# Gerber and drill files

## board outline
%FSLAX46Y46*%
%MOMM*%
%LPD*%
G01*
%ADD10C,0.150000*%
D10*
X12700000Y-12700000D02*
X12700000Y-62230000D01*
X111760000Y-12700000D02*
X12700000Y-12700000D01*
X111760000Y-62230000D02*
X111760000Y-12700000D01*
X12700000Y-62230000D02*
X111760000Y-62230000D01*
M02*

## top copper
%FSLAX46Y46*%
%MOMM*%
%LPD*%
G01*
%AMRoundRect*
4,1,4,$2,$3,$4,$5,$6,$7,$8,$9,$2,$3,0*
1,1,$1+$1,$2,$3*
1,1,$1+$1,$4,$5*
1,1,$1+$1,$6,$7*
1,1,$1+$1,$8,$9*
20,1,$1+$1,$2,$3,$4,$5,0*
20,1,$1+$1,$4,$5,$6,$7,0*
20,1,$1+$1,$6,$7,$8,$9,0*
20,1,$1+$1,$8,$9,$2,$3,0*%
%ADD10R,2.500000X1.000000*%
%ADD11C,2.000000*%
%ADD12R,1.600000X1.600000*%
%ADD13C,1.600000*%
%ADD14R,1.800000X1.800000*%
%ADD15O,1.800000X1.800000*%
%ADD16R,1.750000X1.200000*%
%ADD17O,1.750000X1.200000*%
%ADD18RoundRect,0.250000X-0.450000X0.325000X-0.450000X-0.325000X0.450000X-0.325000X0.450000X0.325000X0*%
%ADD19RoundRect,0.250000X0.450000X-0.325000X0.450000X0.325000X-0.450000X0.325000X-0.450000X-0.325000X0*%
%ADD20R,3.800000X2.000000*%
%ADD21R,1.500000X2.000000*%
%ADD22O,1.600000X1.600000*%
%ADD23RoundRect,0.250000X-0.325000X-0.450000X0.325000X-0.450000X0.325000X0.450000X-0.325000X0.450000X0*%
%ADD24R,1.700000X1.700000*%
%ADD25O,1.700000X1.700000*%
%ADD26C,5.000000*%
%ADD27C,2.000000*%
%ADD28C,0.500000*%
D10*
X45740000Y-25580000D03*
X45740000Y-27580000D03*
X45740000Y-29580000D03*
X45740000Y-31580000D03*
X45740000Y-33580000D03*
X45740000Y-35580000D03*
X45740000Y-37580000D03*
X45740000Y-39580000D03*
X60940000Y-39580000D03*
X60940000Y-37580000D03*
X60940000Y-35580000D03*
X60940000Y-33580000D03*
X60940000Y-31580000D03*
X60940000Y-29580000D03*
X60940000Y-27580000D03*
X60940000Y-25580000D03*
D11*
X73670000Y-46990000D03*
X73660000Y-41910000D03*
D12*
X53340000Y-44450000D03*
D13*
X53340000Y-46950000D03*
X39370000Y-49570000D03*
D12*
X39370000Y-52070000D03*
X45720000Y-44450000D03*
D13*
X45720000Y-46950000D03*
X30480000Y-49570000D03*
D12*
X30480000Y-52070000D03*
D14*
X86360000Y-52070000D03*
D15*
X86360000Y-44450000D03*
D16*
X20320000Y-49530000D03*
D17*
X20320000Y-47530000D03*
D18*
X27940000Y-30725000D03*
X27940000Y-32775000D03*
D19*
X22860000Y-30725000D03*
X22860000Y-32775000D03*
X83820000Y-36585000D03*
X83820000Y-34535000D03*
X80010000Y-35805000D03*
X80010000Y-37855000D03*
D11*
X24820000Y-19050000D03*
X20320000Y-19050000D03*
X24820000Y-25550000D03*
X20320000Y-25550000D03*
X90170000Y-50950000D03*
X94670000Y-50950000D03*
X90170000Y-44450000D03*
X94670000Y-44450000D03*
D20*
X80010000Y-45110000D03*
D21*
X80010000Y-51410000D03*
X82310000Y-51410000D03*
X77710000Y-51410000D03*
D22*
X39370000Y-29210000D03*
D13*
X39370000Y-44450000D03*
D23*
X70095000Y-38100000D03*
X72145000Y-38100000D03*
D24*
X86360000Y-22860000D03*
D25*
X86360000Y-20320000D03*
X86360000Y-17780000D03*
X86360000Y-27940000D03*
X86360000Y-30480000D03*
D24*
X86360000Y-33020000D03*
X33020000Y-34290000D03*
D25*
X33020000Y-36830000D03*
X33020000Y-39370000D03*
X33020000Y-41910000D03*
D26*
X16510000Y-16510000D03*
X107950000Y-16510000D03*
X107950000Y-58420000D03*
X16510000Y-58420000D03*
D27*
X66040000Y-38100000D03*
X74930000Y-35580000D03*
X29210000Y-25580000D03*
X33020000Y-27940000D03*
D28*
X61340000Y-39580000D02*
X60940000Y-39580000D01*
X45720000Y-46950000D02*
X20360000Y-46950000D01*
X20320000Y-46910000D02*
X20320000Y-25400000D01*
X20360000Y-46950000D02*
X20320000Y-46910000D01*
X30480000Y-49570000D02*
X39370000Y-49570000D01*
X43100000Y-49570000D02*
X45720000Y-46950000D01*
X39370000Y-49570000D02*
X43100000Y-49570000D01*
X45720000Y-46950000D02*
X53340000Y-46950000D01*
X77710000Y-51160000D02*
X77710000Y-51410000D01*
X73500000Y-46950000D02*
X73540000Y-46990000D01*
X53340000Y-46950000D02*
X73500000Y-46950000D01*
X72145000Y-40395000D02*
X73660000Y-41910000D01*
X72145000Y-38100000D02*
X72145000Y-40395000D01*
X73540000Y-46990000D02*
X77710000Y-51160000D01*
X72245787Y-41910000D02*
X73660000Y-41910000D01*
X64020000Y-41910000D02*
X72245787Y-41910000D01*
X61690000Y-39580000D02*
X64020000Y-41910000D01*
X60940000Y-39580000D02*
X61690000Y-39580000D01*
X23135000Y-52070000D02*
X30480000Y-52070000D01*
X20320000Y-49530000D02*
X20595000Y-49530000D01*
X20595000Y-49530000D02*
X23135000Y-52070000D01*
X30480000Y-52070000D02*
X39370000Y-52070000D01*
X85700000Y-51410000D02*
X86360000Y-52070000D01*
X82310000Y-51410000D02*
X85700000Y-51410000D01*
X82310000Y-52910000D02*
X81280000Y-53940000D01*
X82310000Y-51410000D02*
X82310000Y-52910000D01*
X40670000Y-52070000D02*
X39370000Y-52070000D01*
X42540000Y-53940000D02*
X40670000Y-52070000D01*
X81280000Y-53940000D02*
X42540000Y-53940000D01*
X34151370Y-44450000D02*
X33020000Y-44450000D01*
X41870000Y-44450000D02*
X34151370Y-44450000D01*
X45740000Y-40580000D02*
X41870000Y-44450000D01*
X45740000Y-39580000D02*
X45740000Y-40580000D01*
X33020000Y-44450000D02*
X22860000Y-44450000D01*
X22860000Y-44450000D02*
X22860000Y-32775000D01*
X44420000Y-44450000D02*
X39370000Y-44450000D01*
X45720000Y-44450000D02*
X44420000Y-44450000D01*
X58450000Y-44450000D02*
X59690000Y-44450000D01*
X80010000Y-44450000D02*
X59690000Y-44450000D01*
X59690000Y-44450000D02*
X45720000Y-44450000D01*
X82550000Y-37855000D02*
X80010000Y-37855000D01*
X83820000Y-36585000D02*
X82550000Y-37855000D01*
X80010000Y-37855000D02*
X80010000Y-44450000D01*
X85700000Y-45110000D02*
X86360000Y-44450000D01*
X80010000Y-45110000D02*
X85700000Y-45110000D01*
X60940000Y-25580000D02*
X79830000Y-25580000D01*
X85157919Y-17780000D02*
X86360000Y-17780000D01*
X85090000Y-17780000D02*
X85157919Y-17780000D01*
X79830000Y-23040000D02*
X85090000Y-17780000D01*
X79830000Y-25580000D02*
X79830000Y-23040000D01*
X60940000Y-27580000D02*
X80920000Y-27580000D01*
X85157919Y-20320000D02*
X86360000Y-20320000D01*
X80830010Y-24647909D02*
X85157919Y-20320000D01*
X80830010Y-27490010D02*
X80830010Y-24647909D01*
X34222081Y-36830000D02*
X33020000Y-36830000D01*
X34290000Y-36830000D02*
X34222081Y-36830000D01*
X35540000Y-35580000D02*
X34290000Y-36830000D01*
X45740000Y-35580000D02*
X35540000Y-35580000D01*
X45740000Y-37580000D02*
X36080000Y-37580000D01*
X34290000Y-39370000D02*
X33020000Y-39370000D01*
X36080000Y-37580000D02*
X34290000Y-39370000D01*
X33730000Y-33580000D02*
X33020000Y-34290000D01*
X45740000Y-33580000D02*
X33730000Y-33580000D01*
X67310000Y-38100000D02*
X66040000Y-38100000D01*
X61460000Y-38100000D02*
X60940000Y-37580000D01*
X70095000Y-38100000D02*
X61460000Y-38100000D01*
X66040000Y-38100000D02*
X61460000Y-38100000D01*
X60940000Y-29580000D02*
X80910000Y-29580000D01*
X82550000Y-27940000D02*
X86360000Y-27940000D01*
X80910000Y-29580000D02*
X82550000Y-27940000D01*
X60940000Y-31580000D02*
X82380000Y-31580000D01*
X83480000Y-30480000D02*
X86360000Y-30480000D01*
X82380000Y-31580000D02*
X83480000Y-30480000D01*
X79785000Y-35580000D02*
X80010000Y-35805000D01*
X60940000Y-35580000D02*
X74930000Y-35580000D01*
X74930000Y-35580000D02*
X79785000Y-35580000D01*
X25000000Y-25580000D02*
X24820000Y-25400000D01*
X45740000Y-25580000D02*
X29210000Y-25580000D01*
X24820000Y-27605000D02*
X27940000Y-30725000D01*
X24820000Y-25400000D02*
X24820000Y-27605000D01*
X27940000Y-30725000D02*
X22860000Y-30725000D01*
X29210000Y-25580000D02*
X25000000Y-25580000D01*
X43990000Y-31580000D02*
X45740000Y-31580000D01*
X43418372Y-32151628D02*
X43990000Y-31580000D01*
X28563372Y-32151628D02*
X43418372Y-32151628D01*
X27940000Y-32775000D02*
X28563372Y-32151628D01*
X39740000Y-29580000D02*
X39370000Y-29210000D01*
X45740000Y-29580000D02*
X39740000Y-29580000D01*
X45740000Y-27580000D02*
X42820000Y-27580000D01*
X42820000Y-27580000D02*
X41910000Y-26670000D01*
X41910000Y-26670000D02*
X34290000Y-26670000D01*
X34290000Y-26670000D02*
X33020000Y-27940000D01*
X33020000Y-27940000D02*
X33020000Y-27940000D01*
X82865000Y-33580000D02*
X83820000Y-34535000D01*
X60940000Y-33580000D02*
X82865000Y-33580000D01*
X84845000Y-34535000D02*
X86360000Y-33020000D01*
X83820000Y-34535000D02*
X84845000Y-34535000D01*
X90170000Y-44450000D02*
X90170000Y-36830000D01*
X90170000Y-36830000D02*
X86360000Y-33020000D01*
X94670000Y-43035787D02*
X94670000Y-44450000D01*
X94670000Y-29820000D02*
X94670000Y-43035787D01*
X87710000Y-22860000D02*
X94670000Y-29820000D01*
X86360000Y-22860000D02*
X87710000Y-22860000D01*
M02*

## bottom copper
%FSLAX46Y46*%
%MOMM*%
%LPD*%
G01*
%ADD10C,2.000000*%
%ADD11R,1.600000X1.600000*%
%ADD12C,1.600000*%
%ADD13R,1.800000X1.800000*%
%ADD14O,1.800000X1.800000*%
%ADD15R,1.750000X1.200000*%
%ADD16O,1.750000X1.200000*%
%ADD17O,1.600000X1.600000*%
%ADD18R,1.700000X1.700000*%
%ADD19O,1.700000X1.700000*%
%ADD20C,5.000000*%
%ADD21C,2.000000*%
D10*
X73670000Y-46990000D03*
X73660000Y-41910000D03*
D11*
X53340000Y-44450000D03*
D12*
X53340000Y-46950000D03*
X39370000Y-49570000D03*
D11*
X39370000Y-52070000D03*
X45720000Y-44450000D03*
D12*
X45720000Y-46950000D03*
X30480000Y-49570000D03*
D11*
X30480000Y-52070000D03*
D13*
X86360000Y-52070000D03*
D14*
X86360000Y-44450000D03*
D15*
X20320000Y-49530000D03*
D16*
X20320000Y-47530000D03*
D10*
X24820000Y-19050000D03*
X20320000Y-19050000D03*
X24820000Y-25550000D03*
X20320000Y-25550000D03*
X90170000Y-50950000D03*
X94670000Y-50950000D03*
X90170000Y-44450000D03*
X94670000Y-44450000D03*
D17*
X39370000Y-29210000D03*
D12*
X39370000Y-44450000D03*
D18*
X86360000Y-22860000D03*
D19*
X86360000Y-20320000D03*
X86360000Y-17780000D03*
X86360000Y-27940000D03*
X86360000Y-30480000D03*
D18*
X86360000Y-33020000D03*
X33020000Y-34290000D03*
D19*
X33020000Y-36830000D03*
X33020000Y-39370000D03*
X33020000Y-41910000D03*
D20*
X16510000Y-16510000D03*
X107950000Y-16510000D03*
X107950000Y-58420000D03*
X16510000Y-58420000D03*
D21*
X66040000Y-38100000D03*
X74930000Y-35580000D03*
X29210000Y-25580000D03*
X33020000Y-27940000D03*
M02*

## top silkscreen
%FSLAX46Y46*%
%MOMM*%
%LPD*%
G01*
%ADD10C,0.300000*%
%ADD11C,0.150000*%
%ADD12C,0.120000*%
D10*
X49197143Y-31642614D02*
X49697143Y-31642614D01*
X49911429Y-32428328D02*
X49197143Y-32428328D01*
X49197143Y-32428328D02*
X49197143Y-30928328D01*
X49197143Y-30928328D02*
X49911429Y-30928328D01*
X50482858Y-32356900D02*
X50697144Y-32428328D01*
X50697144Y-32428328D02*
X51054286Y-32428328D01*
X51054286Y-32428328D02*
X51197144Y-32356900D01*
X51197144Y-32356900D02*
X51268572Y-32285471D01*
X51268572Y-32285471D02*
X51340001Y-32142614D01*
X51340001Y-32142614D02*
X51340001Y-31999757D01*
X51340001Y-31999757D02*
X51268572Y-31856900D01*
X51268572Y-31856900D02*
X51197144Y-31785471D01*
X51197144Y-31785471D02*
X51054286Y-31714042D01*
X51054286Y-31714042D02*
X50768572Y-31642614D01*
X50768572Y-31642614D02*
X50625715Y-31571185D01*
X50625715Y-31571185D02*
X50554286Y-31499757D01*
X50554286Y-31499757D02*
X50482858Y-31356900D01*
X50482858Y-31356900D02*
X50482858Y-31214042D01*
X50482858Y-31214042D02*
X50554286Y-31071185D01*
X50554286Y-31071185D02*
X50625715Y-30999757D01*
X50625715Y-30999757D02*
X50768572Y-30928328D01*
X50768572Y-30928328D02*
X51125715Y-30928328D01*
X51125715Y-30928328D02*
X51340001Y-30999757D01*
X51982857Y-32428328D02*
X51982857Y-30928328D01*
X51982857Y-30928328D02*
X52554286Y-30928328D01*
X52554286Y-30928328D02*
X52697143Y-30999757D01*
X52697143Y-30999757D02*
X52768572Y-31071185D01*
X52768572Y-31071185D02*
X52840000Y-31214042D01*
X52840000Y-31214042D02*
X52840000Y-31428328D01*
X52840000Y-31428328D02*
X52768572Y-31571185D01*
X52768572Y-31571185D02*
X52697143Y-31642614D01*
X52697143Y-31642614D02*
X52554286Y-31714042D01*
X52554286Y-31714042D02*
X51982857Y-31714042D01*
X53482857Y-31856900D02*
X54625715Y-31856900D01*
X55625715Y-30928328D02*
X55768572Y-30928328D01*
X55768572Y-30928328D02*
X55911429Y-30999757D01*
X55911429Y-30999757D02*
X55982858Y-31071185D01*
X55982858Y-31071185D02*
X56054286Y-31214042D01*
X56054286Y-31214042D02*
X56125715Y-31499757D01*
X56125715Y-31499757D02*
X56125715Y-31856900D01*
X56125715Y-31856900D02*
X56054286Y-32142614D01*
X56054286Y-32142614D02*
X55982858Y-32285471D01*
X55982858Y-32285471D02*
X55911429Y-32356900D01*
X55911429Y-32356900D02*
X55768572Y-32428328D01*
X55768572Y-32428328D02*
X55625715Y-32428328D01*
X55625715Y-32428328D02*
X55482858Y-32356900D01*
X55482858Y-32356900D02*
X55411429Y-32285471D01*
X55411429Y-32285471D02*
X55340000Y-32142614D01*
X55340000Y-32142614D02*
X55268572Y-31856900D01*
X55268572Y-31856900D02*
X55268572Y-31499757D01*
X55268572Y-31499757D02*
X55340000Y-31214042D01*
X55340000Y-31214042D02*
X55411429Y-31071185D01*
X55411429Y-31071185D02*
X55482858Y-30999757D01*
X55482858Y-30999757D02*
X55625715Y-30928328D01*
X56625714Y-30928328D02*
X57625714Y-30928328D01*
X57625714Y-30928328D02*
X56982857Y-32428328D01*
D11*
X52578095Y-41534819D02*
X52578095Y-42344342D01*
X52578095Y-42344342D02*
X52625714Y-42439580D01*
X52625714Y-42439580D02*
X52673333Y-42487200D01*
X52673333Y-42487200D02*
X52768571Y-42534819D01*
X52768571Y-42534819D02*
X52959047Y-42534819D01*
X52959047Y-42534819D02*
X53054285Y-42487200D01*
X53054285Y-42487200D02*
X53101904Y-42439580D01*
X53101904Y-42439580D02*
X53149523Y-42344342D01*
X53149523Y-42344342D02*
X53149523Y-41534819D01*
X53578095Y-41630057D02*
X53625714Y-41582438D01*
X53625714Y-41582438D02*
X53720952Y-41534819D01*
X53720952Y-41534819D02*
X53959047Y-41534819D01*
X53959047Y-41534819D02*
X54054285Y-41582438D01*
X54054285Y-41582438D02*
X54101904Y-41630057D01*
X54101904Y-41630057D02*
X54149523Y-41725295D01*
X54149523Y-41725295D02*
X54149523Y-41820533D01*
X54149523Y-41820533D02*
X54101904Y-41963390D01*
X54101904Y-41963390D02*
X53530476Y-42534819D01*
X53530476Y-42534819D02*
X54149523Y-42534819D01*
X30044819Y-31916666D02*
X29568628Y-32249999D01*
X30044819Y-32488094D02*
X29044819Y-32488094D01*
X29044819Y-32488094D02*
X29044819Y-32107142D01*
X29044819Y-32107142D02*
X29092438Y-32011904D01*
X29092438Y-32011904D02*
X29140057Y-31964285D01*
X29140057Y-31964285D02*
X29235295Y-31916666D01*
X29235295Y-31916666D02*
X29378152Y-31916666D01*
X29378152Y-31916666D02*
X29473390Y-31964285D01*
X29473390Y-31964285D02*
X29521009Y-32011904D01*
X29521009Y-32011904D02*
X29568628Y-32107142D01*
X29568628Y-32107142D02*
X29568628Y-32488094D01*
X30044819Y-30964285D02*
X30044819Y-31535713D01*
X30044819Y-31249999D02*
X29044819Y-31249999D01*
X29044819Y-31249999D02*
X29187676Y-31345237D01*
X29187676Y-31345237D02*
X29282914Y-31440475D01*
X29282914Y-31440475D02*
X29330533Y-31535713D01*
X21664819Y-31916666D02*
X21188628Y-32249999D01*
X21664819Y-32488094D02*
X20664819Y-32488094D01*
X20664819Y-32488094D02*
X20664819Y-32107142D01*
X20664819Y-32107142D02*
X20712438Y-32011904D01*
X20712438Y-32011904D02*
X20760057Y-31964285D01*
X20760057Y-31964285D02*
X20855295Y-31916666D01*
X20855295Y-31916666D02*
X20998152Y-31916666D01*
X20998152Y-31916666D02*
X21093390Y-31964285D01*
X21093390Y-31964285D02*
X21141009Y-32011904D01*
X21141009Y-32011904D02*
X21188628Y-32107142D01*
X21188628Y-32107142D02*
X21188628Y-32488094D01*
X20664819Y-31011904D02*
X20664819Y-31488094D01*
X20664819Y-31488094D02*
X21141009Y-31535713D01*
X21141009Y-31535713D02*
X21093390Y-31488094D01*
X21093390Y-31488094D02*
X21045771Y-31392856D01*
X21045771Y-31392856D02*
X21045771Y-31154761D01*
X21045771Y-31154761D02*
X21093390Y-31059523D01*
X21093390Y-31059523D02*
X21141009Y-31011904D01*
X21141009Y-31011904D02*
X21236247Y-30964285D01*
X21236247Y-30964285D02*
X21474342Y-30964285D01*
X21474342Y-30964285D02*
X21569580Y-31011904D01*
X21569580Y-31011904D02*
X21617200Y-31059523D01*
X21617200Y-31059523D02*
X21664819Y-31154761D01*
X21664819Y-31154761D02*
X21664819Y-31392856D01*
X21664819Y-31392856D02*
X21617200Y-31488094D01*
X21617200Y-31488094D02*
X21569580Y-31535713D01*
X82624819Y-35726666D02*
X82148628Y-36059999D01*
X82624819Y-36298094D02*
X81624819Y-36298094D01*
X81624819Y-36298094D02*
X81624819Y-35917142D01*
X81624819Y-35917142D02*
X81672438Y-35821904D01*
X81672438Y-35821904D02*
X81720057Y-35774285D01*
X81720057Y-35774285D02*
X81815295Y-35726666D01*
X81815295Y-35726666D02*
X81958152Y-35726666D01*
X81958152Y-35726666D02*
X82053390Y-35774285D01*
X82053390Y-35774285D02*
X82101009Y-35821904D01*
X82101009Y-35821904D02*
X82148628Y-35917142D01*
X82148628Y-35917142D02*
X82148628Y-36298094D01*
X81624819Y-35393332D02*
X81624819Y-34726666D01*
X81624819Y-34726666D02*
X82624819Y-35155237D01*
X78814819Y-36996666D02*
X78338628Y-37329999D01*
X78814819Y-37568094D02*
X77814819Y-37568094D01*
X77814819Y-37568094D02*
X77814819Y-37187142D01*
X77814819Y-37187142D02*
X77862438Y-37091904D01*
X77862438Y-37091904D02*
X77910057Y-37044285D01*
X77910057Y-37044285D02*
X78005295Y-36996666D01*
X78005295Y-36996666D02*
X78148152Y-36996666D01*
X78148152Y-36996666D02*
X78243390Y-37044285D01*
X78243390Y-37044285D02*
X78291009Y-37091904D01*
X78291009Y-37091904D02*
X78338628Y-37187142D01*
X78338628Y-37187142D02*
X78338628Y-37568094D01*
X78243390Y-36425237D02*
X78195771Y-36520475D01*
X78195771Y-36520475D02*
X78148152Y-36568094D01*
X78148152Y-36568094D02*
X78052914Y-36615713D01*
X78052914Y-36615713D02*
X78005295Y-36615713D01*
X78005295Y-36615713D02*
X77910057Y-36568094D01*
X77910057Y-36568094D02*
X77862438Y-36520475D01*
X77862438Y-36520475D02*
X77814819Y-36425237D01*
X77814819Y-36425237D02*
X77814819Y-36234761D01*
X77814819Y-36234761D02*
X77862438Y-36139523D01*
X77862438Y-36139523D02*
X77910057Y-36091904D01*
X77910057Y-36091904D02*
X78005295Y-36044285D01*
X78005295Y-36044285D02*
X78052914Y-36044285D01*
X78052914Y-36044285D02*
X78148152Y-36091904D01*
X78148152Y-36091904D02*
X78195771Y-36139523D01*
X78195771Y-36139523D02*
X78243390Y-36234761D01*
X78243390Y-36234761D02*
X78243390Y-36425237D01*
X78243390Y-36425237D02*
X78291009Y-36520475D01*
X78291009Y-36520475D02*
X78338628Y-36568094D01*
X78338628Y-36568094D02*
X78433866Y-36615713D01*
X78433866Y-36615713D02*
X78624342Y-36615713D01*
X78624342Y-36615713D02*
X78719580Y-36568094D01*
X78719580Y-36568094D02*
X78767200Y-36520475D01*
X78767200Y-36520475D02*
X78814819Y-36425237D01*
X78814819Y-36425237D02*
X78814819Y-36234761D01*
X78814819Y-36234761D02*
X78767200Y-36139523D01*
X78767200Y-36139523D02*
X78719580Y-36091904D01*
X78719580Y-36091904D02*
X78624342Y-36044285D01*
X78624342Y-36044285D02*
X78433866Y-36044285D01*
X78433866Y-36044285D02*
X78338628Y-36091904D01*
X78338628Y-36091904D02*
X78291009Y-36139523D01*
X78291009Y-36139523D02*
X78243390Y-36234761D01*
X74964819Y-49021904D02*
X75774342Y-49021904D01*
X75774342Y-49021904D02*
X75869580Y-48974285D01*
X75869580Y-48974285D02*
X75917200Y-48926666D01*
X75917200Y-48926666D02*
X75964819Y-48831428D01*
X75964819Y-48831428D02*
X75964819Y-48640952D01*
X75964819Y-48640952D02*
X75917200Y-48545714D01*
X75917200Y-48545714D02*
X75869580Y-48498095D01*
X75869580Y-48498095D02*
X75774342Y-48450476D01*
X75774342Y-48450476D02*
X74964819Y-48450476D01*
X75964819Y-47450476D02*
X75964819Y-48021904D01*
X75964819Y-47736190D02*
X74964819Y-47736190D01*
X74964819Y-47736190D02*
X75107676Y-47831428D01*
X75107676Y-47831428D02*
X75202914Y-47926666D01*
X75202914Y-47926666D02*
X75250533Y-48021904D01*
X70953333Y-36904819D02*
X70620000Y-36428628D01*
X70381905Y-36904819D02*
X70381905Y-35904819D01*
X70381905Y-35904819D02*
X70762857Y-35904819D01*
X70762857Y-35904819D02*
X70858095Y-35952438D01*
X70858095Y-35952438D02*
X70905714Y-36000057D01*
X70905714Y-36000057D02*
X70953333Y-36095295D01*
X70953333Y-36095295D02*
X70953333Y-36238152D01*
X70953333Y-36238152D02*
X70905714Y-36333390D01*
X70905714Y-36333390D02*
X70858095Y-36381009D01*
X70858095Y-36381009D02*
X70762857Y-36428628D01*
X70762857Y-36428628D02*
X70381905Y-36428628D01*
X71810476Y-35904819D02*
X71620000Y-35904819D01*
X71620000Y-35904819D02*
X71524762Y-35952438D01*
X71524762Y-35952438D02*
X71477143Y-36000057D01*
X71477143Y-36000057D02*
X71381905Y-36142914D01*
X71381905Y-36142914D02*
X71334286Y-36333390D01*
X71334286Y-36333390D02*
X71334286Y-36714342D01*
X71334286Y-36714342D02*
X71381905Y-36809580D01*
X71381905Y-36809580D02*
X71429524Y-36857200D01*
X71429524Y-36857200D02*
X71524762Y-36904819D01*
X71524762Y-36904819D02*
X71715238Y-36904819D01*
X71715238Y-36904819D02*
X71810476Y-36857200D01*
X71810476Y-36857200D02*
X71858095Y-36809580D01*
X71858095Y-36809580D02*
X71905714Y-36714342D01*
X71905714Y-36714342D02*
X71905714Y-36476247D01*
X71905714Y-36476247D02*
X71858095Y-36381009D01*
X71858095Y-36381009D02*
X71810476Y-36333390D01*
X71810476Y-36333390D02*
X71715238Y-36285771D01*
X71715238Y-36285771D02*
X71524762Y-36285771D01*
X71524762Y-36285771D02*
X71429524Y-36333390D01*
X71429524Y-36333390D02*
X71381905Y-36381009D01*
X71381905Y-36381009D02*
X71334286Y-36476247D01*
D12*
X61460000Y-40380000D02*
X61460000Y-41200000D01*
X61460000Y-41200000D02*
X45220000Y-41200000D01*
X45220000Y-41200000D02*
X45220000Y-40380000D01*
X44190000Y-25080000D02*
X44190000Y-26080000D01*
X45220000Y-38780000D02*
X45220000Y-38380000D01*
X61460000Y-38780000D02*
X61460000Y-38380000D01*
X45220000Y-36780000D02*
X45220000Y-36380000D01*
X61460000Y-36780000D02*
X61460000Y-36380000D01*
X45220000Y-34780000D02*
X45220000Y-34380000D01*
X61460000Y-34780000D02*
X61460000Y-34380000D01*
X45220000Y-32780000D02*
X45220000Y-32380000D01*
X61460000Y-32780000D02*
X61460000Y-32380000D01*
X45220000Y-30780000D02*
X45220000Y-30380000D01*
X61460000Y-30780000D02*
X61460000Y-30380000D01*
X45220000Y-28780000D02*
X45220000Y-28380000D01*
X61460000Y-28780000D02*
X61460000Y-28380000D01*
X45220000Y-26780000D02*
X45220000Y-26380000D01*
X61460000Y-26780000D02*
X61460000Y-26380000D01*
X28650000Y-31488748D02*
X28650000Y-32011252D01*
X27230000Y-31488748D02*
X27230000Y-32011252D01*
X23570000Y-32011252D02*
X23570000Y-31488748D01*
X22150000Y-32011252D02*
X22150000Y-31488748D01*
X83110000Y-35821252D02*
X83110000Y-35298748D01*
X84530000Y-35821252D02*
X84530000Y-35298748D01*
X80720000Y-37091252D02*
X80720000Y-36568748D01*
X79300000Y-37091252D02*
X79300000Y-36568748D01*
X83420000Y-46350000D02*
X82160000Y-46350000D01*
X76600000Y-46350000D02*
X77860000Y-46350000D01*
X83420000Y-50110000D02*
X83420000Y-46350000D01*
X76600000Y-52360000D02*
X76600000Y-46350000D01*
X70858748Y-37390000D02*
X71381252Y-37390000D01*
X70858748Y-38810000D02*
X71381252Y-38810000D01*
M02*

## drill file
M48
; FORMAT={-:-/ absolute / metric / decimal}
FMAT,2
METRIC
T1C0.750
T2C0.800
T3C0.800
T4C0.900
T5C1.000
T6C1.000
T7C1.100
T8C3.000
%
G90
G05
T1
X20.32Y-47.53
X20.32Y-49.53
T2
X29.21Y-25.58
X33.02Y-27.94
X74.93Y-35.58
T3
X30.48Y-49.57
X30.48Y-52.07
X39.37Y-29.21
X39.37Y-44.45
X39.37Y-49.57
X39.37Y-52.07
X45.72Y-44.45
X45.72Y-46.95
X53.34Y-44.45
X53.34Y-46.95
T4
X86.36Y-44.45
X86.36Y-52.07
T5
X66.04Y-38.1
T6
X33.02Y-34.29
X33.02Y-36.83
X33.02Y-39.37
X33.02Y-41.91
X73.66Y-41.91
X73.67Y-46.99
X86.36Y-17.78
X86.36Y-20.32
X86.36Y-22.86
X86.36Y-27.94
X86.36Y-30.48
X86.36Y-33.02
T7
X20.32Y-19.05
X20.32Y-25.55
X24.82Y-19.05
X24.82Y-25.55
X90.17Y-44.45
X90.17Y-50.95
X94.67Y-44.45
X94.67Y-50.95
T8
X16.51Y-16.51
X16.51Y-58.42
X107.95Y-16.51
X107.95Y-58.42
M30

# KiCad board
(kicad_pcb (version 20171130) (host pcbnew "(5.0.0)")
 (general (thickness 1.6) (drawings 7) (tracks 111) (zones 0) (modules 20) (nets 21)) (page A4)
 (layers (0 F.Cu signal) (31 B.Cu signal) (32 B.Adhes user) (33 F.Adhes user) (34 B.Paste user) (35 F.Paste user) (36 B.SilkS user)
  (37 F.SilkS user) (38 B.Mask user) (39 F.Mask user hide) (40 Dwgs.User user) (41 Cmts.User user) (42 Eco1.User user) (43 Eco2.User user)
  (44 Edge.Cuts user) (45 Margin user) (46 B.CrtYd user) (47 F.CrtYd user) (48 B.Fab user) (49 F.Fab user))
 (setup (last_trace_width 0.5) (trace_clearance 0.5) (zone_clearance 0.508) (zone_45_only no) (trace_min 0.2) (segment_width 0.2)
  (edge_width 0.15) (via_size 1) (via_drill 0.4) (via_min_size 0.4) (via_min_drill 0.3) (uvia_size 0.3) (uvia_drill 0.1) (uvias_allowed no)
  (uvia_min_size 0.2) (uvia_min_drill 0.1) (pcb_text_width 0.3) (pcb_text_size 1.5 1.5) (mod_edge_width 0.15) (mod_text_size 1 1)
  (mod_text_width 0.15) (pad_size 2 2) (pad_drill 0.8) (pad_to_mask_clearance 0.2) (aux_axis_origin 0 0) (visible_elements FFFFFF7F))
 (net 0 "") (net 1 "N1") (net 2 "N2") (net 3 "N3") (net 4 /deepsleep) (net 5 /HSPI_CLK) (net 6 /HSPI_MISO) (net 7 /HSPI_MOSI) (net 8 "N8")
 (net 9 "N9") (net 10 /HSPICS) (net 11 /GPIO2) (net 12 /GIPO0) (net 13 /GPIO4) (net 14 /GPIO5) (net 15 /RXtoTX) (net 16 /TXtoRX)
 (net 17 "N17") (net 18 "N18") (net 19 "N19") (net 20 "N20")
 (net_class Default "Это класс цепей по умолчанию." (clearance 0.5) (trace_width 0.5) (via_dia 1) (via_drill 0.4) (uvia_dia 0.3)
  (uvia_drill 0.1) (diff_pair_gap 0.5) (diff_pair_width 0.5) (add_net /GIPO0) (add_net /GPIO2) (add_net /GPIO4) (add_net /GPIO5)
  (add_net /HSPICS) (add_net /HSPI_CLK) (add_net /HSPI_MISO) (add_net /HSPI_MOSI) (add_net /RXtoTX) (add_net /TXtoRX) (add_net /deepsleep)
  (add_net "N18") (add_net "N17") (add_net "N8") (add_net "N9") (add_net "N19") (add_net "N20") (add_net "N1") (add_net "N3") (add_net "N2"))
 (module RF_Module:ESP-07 (layer F.Cu) (at 53.34 30.48)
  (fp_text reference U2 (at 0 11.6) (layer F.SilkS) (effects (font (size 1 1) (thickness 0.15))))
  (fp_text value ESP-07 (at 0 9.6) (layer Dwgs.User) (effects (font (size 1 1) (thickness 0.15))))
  (fp_line (start 8.12 9.9) (end 8.12 10.72) (layer F.SilkS) (width 0.12))
  (fp_line (start 8.12 10.72) (end -8.12 10.72) (layer F.SilkS) (width 0.12))
  (fp_line (start -8.12 10.72) (end -8.12 9.9) (layer F.SilkS) (width 0.12))
  (fp_line (start -9.15 -5.4) (end -9.15 -4.4) (layer F.SilkS) (width 0.12))
  (fp_line (start -8.12 8.3) (end -8.12 7.9) (layer F.SilkS) (width 0.12))
  (fp_line (start 8.12 8.3) (end 8.12 7.9) (layer F.SilkS) (width 0.12))
  (fp_line (start -8.12 6.3) (end -8.12 5.9) (layer F.SilkS) (width 0.12))
  (fp_line (start 8.12 6.3) (end 8.12 5.9) (layer F.SilkS) (width 0.12))
  (fp_line (start -8.12 4.3) (end -8.12 3.9) (layer F.SilkS) (width 0.12))
  (fp_line (start 8.12 4.3) (end 8.12 3.9) (layer F.SilkS) (width 0.12))
  (fp_line (start -8.12 2.3) (end -8.12 1.9) (layer F.SilkS) (width 0.12))
  (fp_line (start 8.12 2.3) (end 8.12 1.9) (layer F.SilkS) (width 0.12))
  (fp_line (start -8.12 0.3) (end -8.12 -0.1) (layer F.SilkS) (width 0.12))
  (fp_line (start 8.12 0.3) (end 8.12 -0.1) (layer F.SilkS) (width 0.12))
  (fp_line (start -8.12 -1.7) (end -8.12 -2.1) (layer F.SilkS) (width 0.12))
  (fp_line (start 8.12 -1.7) (end 8.12 -2.1) (layer F.SilkS) (width 0.12))
  (fp_line (start -8.12 -3.7) (end -8.12 -4.1) (layer F.SilkS) (width 0.12))
  (fp_line (start 8.12 -3.7) (end 8.12 -4.1) (layer F.SilkS) (width 0.12))
  (pad 1 smd rect (at -7.6 -4.9) (size 2.5 1) (layers F.Cu F.Paste F.Mask) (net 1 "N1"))
  (pad 2 smd rect (at -7.6 -2.9) (size 2.5 1) (layers F.Cu F.Paste F.Mask) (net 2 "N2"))
  (pad 3 smd rect (at -7.6 -0.9) (size 2.5 1) (layers F.Cu F.Paste F.Mask) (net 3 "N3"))
  (pad 4 smd rect (at -7.6 1.1) (size 2.5 1) (layers F.Cu F.Paste F.Mask) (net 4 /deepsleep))
  (pad 5 smd rect (at -7.6 3.1) (size 2.5 1) (layers F.Cu F.Paste F.Mask) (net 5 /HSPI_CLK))
  (pad 6 smd rect (at -7.6 5.1) (size 2.5 1) (layers F.Cu F.Paste F.Mask) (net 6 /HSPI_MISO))
  (pad 7 smd rect (at -7.6 7.1) (size 2.5 1) (layers F.Cu F.Paste F.Mask) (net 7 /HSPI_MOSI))
  (pad 8 smd rect (at -7.6 9.1) (size 2.5 1) (layers F.Cu F.Paste F.Mask) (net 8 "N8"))
  (pad 9 smd rect (at 7.6 9.1) (size 2.5 1) (layers F.Cu F.Paste F.Mask) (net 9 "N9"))
  (pad 10 smd rect (at 7.6 7.1) (size 2.5 1) (layers F.Cu F.Paste F.Mask) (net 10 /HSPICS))
  (pad 11 smd rect (at 7.6 5.1) (size 2.5 1) (layers F.Cu F.Paste F.Mask) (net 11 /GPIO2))
  (pad 12 smd rect (at 7.6 3.1) (size 2.5 1) (layers F.Cu F.Paste F.Mask) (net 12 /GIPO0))
  (pad 13 smd rect (at 7.6 1.1) (size 2.5 1) (layers F.Cu F.Paste F.Mask) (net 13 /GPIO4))
  (pad 14 smd rect (at 7.6 -0.9) (size 2.5 1) (layers F.Cu F.Paste F.Mask) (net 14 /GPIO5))
  (pad 15 smd rect (at 7.6 -2.9) (size 2.5 1) (layers F.Cu F.Paste F.Mask) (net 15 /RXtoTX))
  (pad 16 smd rect (at 7.6 -4.9) (size 2.5 1) (layers F.Cu F.Paste F.Mask) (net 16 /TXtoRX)))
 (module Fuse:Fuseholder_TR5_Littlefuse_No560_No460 (layer B.Cu) (at 73.66 41.91 270)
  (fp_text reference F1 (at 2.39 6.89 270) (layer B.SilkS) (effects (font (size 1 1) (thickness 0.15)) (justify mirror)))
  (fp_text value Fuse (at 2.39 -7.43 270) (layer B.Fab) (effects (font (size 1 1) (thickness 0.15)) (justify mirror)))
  (pad 2 thru_hole circle (at 5.08 -0.01 270) (size 2 2) (drill 1) (layers *.Cu *.Mask) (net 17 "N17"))
  (pad 1 thru_hole circle (at 0 0 270) (size 2 2) (drill 1) (layers *.Cu *.Mask) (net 9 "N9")))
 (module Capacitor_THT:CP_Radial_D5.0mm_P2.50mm (layer B.Cu) (at 53.34 44.45 270)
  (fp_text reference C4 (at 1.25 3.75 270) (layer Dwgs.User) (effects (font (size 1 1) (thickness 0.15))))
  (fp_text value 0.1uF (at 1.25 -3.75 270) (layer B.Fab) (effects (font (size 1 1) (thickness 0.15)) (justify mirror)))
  (pad 1 thru_hole rect (at 0 0 270) (size 1.6 1.6) (drill 0.8) (layers *.Cu *.Mask) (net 8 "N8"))
  (pad 2 thru_hole circle (at 2.5 0 270) (size 1.6 1.6) (drill 0.8) (layers *.Cu *.Mask) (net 17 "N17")))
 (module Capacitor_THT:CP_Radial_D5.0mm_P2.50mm (layer B.Cu) (at 39.37 52.07 90)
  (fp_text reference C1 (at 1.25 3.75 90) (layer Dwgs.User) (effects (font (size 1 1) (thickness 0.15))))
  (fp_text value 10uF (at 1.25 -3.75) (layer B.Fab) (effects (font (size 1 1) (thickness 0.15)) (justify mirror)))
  (pad 2 thru_hole circle (at 2.5 0 90) (size 1.6 1.6) (drill 0.8) (layers *.Cu *.Mask) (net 17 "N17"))
  (pad 1 thru_hole rect (at 0 0 90) (size 1.6 1.6) (drill 0.8) (layers *.Cu *.Mask) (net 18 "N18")))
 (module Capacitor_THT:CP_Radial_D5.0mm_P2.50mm (layer B.Cu) (at 45.72 44.45 270)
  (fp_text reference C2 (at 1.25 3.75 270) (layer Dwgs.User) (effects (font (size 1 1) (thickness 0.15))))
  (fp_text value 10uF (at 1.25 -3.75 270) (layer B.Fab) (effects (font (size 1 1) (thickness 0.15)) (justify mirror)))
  (pad 1 thru_hole rect (at 0 0 270) (size 1.6 1.6) (drill 0.8) (layers *.Cu *.Mask) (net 8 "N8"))
  (pad 2 thru_hole circle (at 2.5 0 270) (size 1.6 1.6) (drill 0.8) (layers *.Cu *.Mask) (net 17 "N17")))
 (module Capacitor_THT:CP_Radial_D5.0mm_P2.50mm (layer B.Cu) (at 30.48 52.07 90)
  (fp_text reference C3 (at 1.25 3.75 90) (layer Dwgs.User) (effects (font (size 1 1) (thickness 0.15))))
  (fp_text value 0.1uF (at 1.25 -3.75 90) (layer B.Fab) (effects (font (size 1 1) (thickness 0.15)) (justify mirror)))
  (pad 2 thru_hole circle (at 2.5 0 90) (size 1.6 1.6) (drill 0.8) (layers *.Cu *.Mask) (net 17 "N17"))
  (pad 1 thru_hole rect (at 0 0 90) (size 1.6 1.6) (drill 0.8) (layers *.Cu *.Mask) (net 18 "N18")))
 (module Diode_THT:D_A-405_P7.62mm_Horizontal (layer B.Cu) (at 86.36 52.07 90)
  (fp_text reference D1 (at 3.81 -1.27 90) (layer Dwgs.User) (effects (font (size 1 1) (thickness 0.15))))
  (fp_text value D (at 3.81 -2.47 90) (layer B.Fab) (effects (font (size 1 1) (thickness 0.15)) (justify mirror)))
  (pad 1 thru_hole rect (at 0 0 90) (size 1.8 1.8) (drill 0.9) (layers *.Cu *.Mask) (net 18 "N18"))
  (pad 2 thru_hole oval (at 7.62 0 90) (size 1.8 1.8) (drill 0.9) (layers *.Cu *.Mask) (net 8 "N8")))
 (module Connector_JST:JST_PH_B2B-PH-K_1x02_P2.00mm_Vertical (layer B.Cu) (at 20.32 49.53 90)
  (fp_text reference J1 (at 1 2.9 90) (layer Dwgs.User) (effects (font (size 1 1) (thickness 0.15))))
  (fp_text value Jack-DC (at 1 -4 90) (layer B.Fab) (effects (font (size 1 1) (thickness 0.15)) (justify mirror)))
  (pad 1 thru_hole rect (at 0 0 90) (size 1.2 1.75) (drill 0.75) (layers *.Cu *.Mask) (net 18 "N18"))
  (pad 2 thru_hole oval (at 2 0 90) (size 1.2 1.75) (drill 0.75) (layers *.Cu *.Mask) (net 17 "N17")))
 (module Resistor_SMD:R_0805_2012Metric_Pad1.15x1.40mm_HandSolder (layer F.Cu) (at 27.94 31.75 270)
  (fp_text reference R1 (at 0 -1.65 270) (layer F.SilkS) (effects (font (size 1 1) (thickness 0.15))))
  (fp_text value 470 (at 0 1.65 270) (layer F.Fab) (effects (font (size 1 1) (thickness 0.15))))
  (fp_line (start -0.261252 -0.71) (end 0.261252 -0.71) (layer F.SilkS) (width 0.12))
  (fp_line (start -0.261252 0.71) (end 0.261252 0.71) (layer F.SilkS) (width 0.12))
  (pad 1 smd roundrect (at -1.025 0 270) (size 1.15 1.4) (layers F.Cu F.Paste F.Mask) (roundrect_rratio 0.217391) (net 1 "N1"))
  (pad 2 smd roundrect (at 1.025 0 270) (size 1.15 1.4) (layers F.Cu F.Paste F.Mask) (roundrect_rratio 0.217391) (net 4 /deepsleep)))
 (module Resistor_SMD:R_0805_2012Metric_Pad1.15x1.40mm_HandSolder (layer F.Cu) (at 22.86 31.75 90)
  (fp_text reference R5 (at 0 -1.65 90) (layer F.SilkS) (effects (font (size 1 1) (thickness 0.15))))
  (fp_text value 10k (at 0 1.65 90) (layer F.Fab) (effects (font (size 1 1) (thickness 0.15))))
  (fp_line (start -0.261252 0.71) (end 0.261252 0.71) (layer F.SilkS) (width 0.12))
  (fp_line (start -0.261252 -0.71) (end 0.261252 -0.71) (layer F.SilkS) (width 0.12))
  (pad 2 smd roundrect (at 1.025 0 90) (size 1.15 1.4) (layers F.Cu F.Paste F.Mask) (roundrect_rratio 0.217391) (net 1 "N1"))
  (pad 1 smd roundrect (at -1.025 0 90) (size 1.15 1.4) (layers F.Cu F.Paste F.Mask) (roundrect_rratio 0.217391) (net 8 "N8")))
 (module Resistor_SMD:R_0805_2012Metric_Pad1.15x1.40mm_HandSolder (layer F.Cu) (at 83.82 35.56 90)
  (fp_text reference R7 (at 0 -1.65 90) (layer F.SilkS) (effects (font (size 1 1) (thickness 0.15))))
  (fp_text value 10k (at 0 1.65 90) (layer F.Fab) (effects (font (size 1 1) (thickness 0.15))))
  (fp_line (start -0.261252 -0.71) (end 0.261252 -0.71) (layer F.SilkS) (width 0.12))
  (fp_line (start -0.261252 0.71) (end 0.261252 0.71) (layer F.SilkS) (width 0.12))
  (pad 1 smd roundrect (at -1.025 0 90) (size 1.15 1.4) (layers F.Cu F.Paste F.Mask) (roundrect_rratio 0.217391) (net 8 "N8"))
  (pad 2 smd roundrect (at 1.025 0 90) (size 1.15 1.4) (layers F.Cu F.Paste F.Mask) (roundrect_rratio 0.217391) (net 12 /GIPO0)))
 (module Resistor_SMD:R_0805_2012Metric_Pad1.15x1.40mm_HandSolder (layer F.Cu) (at 80.01 36.83 90)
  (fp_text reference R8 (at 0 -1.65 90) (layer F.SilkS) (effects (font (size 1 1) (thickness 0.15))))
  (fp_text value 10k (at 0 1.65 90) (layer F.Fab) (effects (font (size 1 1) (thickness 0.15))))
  (fp_line (start -0.261252 0.71) (end 0.261252 0.71) (layer F.SilkS) (width 0.12))
  (fp_line (start -0.261252 -0.71) (end 0.261252 -0.71) (layer F.SilkS) (width 0.12))
  (pad 2 smd roundrect (at 1.025 0 90) (size 1.15 1.4) (layers F.Cu F.Paste F.Mask) (roundrect_rratio 0.217391) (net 11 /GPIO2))
  (pad 1 smd roundrect (at -1.025 0 90) (size 1.15 1.4) (layers F.Cu F.Paste F.Mask) (roundrect_rratio 0.217391) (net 8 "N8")))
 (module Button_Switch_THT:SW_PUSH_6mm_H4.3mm (layer B.Cu) (at 20.32 19.05 270)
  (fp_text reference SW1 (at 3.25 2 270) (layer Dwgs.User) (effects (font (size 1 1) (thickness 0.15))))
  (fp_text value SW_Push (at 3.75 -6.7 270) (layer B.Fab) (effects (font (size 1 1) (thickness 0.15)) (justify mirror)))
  (pad 2 thru_hole circle (at 0 -4.5 180) (size 2 2) (drill 1.1) (layers *.Cu *.Mask) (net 1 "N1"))
  (pad 1 thru_hole circle (at 0 0 180) (size 2 2) (drill 1.1) (layers *.Cu *.Mask) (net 17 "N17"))
  (pad 2 thru_hole circle (at 6.5 -4.5 180) (size 2 2) (drill 1.1) (layers *.Cu *.Mask) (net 1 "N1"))
  (pad 1 thru_hole circle (at 6.5 0 180) (size 2 2) (drill 1.1) (layers *.Cu *.Mask) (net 17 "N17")))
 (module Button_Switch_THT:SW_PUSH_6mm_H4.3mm (layer B.Cu) (at 90.17 44.45 270)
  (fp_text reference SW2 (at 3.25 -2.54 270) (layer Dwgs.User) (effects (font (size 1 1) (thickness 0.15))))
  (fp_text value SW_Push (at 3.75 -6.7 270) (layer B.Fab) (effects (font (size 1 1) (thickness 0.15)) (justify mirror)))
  (pad 1 thru_hole circle (at 6.5 0 180) (size 2 2) (drill 1.1) (layers *.Cu *.Mask) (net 12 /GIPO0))
  (pad 2 thru_hole circle (at 6.5 -4.5 180) (size 2 2) (drill 1.1) (layers *.Cu *.Mask) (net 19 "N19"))
  (pad 1 thru_hole circle (at 0 0 180) (size 2 2) (drill 1.1) (layers *.Cu *.Mask) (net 12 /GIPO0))
  (pad 2 thru_hole circle (at 0 -4.5 180) (size 2 2) (drill 1.1) (layers *.Cu *.Mask) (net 19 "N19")))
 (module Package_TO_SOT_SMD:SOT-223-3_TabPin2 (layer F.Cu) (at 80.01 48.26 90)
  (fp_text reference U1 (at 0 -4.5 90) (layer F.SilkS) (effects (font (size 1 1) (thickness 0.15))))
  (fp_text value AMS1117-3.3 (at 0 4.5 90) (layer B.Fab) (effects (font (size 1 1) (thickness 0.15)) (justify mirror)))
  (fp_line (start 1.91 3.41) (end 1.91 2.15) (layer F.SilkS) (width 0.12))
  (fp_line (start 1.91 -3.41) (end 1.91 -2.15) (layer F.SilkS) (width 0.12))
  (fp_line (start -1.85 3.41) (end 1.91 3.41) (layer F.SilkS) (width 0.12))
  (fp_line (start -4.1 -3.41) (end 1.91 -3.41) (layer F.SilkS) (width 0.12))
  (pad 2 smd rect (at 3.15 0 90) (size 2 3.8) (layers F.Cu F.Paste F.Mask) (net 8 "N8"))
  (pad 2 smd rect (at -3.15 0 90) (size 2 1.5) (layers F.Cu F.Paste F.Mask) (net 8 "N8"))
  (pad 3 smd rect (at -3.15 2.3 90) (size 2 1.5) (layers F.Cu F.Paste F.Mask) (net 18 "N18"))
  (pad 1 smd rect (at -3.15 -2.3 90) (size 2 1.5) (layers F.Cu F.Paste F.Mask) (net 17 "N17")))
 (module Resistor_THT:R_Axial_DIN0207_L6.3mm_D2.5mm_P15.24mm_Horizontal (layer B.Cu) (at 39.37 44.45 90)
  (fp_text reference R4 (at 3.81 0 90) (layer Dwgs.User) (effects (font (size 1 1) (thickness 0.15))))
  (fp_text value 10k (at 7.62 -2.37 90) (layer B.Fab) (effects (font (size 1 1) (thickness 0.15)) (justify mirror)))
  (pad 2 thru_hole oval (at 15.24 0 90) (size 1.6 1.6) (drill 0.8) (layers *.Cu *.Mask) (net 3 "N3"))
  (pad 1 thru_hole circle (at 0 0 90) (size 1.6 1.6) (drill 0.8) (layers *.Cu *.Mask) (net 8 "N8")))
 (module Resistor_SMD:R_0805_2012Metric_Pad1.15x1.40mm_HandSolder (layer F.Cu) (at 71.12 38.1)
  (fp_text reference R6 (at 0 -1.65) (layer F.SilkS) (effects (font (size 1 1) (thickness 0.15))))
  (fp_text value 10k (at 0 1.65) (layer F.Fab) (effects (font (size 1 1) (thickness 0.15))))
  (fp_line (start -0.261252 -0.71) (end 0.261252 -0.71) (layer F.SilkS) (width 0.12))
  (fp_line (start -0.261252 0.71) (end 0.261252 0.71) (layer F.SilkS) (width 0.12))
  (pad 1 smd roundrect (at -1.025 0) (size 1.15 1.4) (layers F.Cu F.Paste F.Mask) (roundrect_rratio 0.217391) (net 10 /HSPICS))
  (pad 2 smd roundrect (at 1.025 0) (size 1.15 1.4) (layers F.Cu F.Paste F.Mask) (roundrect_rratio 0.217391) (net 9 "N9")))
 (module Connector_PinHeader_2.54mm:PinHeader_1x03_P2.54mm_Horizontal (layer B.Cu) (at 86.36 22.86)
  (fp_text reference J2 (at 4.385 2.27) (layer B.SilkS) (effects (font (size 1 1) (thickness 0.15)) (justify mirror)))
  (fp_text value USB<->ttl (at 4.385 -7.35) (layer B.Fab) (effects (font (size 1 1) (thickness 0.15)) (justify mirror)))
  (pad 1 thru_hole rect (at 0 0) (size 1.7 1.7) (drill 1) (layers *.Cu *.Mask) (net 19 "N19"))
  (pad 2 thru_hole oval (at 0 -2.54) (size 1.7 1.7) (drill 1) (layers *.Cu *.Mask) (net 15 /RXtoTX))
  (pad 3 thru_hole oval (at 0 -5.08) (size 1.7 1.7) (drill 1) (layers *.Cu *.Mask) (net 16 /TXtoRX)))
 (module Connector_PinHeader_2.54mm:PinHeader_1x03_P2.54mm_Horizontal (layer B.Cu) (at 86.36 33.02)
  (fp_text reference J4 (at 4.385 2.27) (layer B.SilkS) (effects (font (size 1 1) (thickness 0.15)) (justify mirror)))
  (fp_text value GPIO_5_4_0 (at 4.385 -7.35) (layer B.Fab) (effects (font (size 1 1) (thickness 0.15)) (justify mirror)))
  (pad 3 thru_hole oval (at 0 -5.08) (size 1.7 1.7) (drill 1) (layers *.Cu *.Mask) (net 14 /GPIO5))
  (pad 2 thru_hole oval (at 0 -2.54) (size 1.7 1.7) (drill 1) (layers *.Cu *.Mask) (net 13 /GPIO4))
  (pad 1 thru_hole rect (at 0 0) (size 1.7 1.7) (drill 1) (layers *.Cu *.Mask) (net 12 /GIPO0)))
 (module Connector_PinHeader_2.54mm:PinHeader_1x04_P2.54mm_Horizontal (layer B.Cu) (at 33.02 34.29 180)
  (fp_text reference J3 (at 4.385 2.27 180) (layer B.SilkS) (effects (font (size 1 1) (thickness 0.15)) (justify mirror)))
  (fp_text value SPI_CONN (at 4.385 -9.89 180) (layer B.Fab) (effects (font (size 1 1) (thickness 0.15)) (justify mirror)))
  (pad 1 thru_hole rect (at 0 0 180) (size 1.7 1.7) (drill 1) (layers *.Cu *.Mask) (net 5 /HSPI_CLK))
  (pad 2 thru_hole oval (at 0 -2.54 180) (size 1.7 1.7) (drill 1) (layers *.Cu *.Mask) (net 6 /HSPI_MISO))
  (pad 3 thru_hole oval (at 0 -5.08 180) (size 1.7 1.7) (drill 1) (layers *.Cu *.Mask) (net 7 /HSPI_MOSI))
  (pad 4 thru_hole oval (at 0 -7.62 180) (size 1.7 1.7) (drill 1) (layers *.Cu *.Mask) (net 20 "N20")))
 (gr_line (start 12.7 12.7) (end 12.7 62.23) (layer Edge.Cuts) (width 0.15))
 (gr_line (start 111.76 12.7) (end 12.7 12.7) (layer Edge.Cuts) (width 0.15))
 (gr_line (start 111.76 62.23) (end 111.76 12.7) (layer Edge.Cuts) (width 0.15))
 (gr_line (start 12.7 62.23) (end 111.76 62.23) (layer Edge.Cuts) (width 0.15))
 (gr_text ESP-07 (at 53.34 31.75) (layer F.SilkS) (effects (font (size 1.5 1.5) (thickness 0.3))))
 (via (at 16.51 16.51) (size 5) (drill 3) (layers F.Cu B.Cu) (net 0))
 (via (at 107.95 16.51) (size 5) (drill 3) (layers F.Cu B.Cu) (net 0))
 (via (at 107.95 58.42) (size 5) (drill 3) (layers F.Cu B.Cu) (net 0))
 (via (at 16.51 58.42) (size 5) (drill 3) (layers F.Cu B.Cu) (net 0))
 (segment (start 61.34 39.58) (end 60.94 39.58) (width 0.5) (layer F.Cu) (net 9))
 (segment (start 45.72 46.95) (end 20.36 46.95) (width 0.5) (layer F.Cu) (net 17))
 (segment (start 20.32 46.91) (end 20.32 25.4) (width 0.5) (layer F.Cu) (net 17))
 (segment (start 20.36 46.95) (end 20.32 46.91) (width 0.5) (layer F.Cu) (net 17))
 (segment (start 30.48 49.57) (end 39.37 49.57) (width 0.5) (layer F.Cu) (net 17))
 (segment (start 43.1 49.57) (end 45.72 46.95) (width 0.5) (layer F.Cu) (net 17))
 (segment (start 39.37 49.57) (end 43.1 49.57) (width 0.5) (layer F.Cu) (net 17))
 (segment (start 45.72 46.95) (end 53.34 46.95) (width 0.5) (layer F.Cu) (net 17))
 (segment (start 77.71 51.16) (end 77.71 51.41) (width 0.5) (layer F.Cu) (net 17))
 (segment (start 73.5 46.95) (end 73.54 46.99) (width 0.5) (layer F.Cu) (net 17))
 (segment (start 53.34 46.95) (end 73.5 46.95) (width 0.5) (layer F.Cu) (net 17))
 (segment (start 72.145 40.395) (end 73.66 41.91) (width 0.5) (layer F.Cu) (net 9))
 (segment (start 72.145 38.1) (end 72.145 40.395) (width 0.5) (layer F.Cu) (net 9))
 (segment (start 73.54 46.99) (end 77.71 51.16) (width 0.5) (layer F.Cu) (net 17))
 (segment (start 72.245787 41.91) (end 73.66 41.91) (width 0.5) (layer F.Cu) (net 9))
 (segment (start 64.02 41.91) (end 72.245787 41.91) (width 0.5) (layer F.Cu) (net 9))
 (segment (start 61.69 39.58) (end 64.02 41.91) (width 0.5) (layer F.Cu) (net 9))
 (segment (start 60.94 39.58) (end 61.69 39.58) (width 0.5) (layer F.Cu) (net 9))
 (segment (start 23.135 52.07) (end 30.48 52.07) (width 0.5) (layer F.Cu) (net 18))
 (segment (start 20.32 49.53) (end 20.595 49.53) (width 0.5) (layer F.Cu) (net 18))
 (segment (start 20.595 49.53) (end 23.135 52.07) (width 0.5) (layer F.Cu) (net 18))
 (segment (start 30.48 52.07) (end 39.37 52.07) (width 0.5) (layer F.Cu) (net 18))
 (segment (start 85.7 51.41) (end 86.36 52.07) (width 0.5) (layer F.Cu) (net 18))
 (segment (start 82.31 51.41) (end 85.7 51.41) (width 0.5) (layer F.Cu) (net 18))
 (segment (start 82.31 52.91) (end 81.28 53.94) (width 0.5) (layer F.Cu) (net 18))
 (segment (start 82.31 51.41) (end 82.31 52.91) (width 0.5) (layer F.Cu) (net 18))
 (segment (start 40.67 52.07) (end 39.37 52.07) (width 0.5) (layer F.Cu) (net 18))
 (segment (start 42.54 53.94) (end 40.67 52.07) (width 0.5) (layer F.Cu) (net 18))
 (segment (start 81.28 53.94) (end 42.54 53.94) (width 0.5) (layer F.Cu) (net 18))
 (segment (start 34.15137 44.45) (end 33.02 44.45) (width 0.5) (layer F.Cu) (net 8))
 (segment (start 41.87 44.45) (end 34.15137 44.45) (width 0.5) (layer F.Cu) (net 8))
 (segment (start 45.74 40.58) (end 41.87 44.45) (width 0.5) (layer F.Cu) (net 8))
 (segment (start 45.74 39.58) (end 45.74 40.58) (width 0.5) (layer F.Cu) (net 8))
 (segment (start 33.02 44.45) (end 22.86 44.45) (width 0.5) (layer F.Cu) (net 8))
 (segment (start 22.86 44.45) (end 22.86 32.775) (width 0.5) (layer F.Cu) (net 8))
 (segment (start 44.42 44.45) (end 39.37 44.45) (width 0.5) (layer F.Cu) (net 8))
 (segment (start 45.72 44.45) (end 44.42 44.45) (width 0.5) (layer F.Cu) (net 8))
 (segment (start 58.45 44.45) (end 59.69 44.45) (width 0.5) (layer F.Cu) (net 8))
 (segment (start 80.01 44.45) (end 59.69 44.45) (width 0.5) (layer F.Cu) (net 8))
 (segment (start 59.69 44.45) (end 45.72 44.45) (width 0.5) (layer F.Cu) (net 8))
 (segment (start 82.55 37.855) (end 80.01 37.855) (width 0.5) (layer F.Cu) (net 8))
 (segment (start 83.82 36.585) (end 82.55 37.855) (width 0.5) (layer F.Cu) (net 8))
 (segment (start 80.01 37.855) (end 80.01 44.45) (width 0.5) (layer F.Cu) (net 8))
 (segment (start 85.7 45.11) (end 86.36 44.45) (width 0.5) (layer F.Cu) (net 8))
 (segment (start 80.01 45.11) (end 85.7 45.11) (width 0.5) (layer F.Cu) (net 8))
 (segment (start 60.94 25.58) (end 79.83 25.58) (width 0.5) (layer F.Cu) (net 16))
 (segment (start 85.157919 17.78) (end 86.36 17.78) (width 0.5) (layer F.Cu) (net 16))
 (segment (start 85.09 17.78) (end 85.157919 17.78) (width 0.5) (layer F.Cu) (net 16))
 (segment (start 79.83 23.04) (end 85.09 17.78) (width 0.5) (layer F.Cu) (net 16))
 (segment (start 79.83 25.58) (end 79.83 23.04) (width 0.5) (layer F.Cu) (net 16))
 (segment (start 60.94 27.58) (end 80.92 27.58) (width 0.5) (layer F.Cu) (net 15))
 (segment (start 85.157919 20.32) (end 86.36 20.32) (width 0.5) (layer F.Cu) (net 15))
 (segment (start 80.83001 24.647909) (end 85.157919 20.32) (width 0.5) (layer F.Cu) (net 15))
 (segment (start 80.83001 27.49001) (end 80.83001 24.647909) (width 0.5) (layer F.Cu) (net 15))
 (segment (start 34.222081 36.83) (end 33.02 36.83) (width 0.5) (layer F.Cu) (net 6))
 (segment (start 34.29 36.83) (end 34.222081 36.83) (width 0.5) (layer F.Cu) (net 6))
 (segment (start 35.54 35.58) (end 34.29 36.83) (width 0.5) (layer F.Cu) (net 6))
 (segment (start 45.74 35.58) (end 35.54 35.58) (width 0.5) (layer F.Cu) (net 6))
 (segment (start 45.74 37.58) (end 36.08 37.58) (width 0.5) (layer F.Cu) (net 7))
 (segment (start 34.29 39.37) (end 33.02 39.37) (width 0.5) (layer F.Cu) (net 7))
 (segment (start 36.08 37.58) (end 34.29 39.37) (width 0.5) (layer F.Cu) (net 7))
 (segment (start 33.73 33.58) (end 33.02 34.29) (width 0.5) (layer F.Cu) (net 5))
 (segment (start 45.74 33.58) (end 33.73 33.58) (width 0.5) (layer F.Cu) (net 5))
 (segment (start 67.31 38.1) (end 66.04 38.1) (width 0.5) (layer F.Cu) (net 10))
 (segment (start 61.46 38.1) (end 60.94 37.58) (width 0.5) (layer F.Cu) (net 10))
 (segment (start 70.095 38.1) (end 61.46 38.1) (width 0.5) (layer F.Cu) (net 10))
 (segment (start 66.04 38.1) (end 61.46 38.1) (width 0.5) (layer F.Cu) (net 10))
 (via (at 66.04 38.1) (size 2) (drill 1) (layers F.Cu B.Cu) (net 10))
 (segment (start 60.94 29.58) (end 80.91 29.58) (width 0.5) (layer F.Cu) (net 14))
 (segment (start 82.55 27.94) (end 86.36 27.94) (width 0.5) (layer F.Cu) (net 14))
 (segment (start 80.91 29.58) (end 82.55 27.94) (width 0.5) (layer F.Cu) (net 14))
 (segment (start 60.94 31.58) (end 82.38 31.58) (width 0.5) (layer F.Cu) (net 13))
 (segment (start 83.48 30.48) (end 86.36 30.48) (width 0.5) (layer F.Cu) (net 13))
 (segment (start 82.38 31.58) (end 83.48 30.48) (width 0.5) (layer F.Cu) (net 13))
 (segment (start 79.785 35.58) (end 80.01 35.805) (width 0.5) (layer F.Cu) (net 11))
 (segment (start 60.94 35.58) (end 74.93 35.58) (width 0.5) (layer F.Cu) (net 11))
 (segment (start 74.93 35.58) (end 79.785 35.58) (width 0.5) (layer F.Cu) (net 11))
 (via (at 74.93 35.58) (size 2) (drill 0.8) (layers F.Cu B.Cu) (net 11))
 (segment (start 25 25.58) (end 24.82 25.4) (width 0.5) (layer F.Cu) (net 1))
 (segment (start 45.74 25.58) (end 29.21 25.58) (width 0.5) (layer F.Cu) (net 1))
 (segment (start 24.82 27.605) (end 27.94 30.725) (width 0.5) (layer F.Cu) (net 1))
 (segment (start 24.82 25.4) (end 24.82 27.605) (width 0.5) (layer F.Cu) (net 1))
 (segment (start 27.94 30.725) (end 22.86 30.725) (width 0.5) (layer F.Cu) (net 1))
 (segment (start 29.21 25.58) (end 25 25.58) (width 0.5) (layer F.Cu) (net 1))
 (via (at 29.21 25.58) (size 2) (drill 0.8) (layers F.Cu B.Cu) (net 1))
 (segment (start 43.99 31.58) (end 45.74 31.58) (width 0.5) (layer F.Cu) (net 4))
 (segment (start 43.418372 32.151628) (end 43.99 31.58) (width 0.5) (layer F.Cu) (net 4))
 (segment (start 28.563372 32.151628) (end 43.418372 32.151628) (width 0.5) (layer F.Cu) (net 4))
 (segment (start 27.94 32.775) (end 28.563372 32.151628) (width 0.5) (layer F.Cu) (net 4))
 (segment (start 39.74 29.58) (end 39.37 29.21) (width 0.5) (layer F.Cu) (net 3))
 (segment (start 45.74 29.58) (end 39.74 29.58) (width 0.5) (layer F.Cu) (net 3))
 (segment (start 45.74 27.58) (end 42.82 27.58) (width 0.5) (layer F.Cu) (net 2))
 (segment (start 42.82 27.58) (end 41.91 26.67) (width 0.5) (layer F.Cu) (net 2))
 (segment (start 41.91 26.67) (end 34.29 26.67) (width 0.5) (layer F.Cu) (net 2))
 (segment (start 34.29 26.67) (end 33.02 27.94) (width 0.5) (layer F.Cu) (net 2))
 (segment (start 33.02 27.94) (end 33.02 27.94) (width 0.5) (layer F.Cu) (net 2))
 (via (at 33.02 27.94) (size 2) (drill 0.8) (layers F.Cu B.Cu) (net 2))
 (segment (start 82.865 33.58) (end 83.82 34.535) (width 0.5) (layer F.Cu) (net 12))
 (segment (start 60.94 33.58) (end 82.865 33.58) (width 0.5) (layer F.Cu) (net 12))
 (segment (start 84.845 34.535) (end 86.36 33.02) (width 0.5) (layer F.Cu) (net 12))
 (segment (start 83.82 34.535) (end 84.845 34.535) (width 0.5) (layer F.Cu) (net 12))
 (segment (start 90.17 44.45) (end 90.17 36.83) (width 0.5) (layer F.Cu) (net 12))
 (segment (start 90.17 36.83) (end 86.36 33.02) (width 0.5) (layer F.Cu) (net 12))
 (segment (start 94.67 43.035787) (end 94.67 44.45) (width 0.5) (layer F.Cu) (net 19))
 (segment (start 94.67 29.82) (end 94.67 43.035787) (width 0.5) (layer F.Cu) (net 19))
 (segment (start 87.71 22.86) (end 94.67 29.82) (width 0.5) (layer F.Cu) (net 19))
 (segment (start 86.36 22.86) (end 87.71 22.86) (width 0.5) (layer F.Cu) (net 19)))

